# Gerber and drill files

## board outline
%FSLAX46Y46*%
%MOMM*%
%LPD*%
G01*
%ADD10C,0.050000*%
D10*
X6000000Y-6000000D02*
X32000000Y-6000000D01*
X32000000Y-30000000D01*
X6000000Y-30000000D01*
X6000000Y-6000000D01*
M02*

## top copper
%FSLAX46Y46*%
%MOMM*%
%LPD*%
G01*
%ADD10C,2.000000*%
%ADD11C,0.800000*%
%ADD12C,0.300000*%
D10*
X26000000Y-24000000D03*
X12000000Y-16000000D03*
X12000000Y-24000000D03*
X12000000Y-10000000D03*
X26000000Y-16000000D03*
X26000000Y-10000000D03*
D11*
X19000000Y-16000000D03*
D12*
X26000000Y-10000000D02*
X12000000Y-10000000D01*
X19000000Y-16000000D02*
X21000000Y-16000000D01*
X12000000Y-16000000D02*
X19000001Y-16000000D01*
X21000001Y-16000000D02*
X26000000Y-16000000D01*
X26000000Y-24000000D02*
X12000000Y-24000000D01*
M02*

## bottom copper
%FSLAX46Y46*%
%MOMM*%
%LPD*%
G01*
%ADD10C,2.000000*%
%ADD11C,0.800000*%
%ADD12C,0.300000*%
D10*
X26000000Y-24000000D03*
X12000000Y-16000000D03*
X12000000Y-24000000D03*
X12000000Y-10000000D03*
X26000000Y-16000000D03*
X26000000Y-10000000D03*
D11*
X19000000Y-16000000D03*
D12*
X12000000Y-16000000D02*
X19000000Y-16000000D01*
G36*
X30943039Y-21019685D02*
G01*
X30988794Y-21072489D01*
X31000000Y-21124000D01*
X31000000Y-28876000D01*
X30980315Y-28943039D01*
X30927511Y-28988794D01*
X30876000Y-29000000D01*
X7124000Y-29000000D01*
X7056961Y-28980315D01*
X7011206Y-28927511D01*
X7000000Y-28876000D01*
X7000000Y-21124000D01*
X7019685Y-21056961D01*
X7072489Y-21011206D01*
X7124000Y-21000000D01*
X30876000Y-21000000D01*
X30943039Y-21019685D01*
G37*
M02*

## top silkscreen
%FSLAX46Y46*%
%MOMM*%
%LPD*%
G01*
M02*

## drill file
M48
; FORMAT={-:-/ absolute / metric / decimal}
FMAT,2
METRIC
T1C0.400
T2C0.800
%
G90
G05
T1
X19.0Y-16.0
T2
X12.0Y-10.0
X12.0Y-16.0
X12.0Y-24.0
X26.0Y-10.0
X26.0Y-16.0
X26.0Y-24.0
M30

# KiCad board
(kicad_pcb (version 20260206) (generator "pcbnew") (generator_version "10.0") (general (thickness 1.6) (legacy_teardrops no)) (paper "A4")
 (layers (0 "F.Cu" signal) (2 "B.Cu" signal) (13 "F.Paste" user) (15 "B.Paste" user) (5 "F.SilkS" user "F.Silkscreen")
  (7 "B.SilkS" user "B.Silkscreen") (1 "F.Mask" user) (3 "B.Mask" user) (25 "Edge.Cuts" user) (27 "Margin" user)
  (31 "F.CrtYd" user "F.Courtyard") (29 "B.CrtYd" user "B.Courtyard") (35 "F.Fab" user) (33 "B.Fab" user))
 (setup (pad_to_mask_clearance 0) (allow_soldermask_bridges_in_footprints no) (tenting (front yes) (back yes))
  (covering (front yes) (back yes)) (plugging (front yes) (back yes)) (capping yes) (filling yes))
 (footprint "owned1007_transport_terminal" (layer "F.Cu") (at 26 24)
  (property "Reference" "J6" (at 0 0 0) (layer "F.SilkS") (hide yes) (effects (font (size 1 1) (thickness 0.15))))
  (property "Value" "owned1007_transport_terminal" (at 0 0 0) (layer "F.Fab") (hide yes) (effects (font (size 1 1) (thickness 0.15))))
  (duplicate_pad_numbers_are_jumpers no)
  (pad "1" thru_hole circle (at 0 0) (size 2 2) (drill 0.8) (layers "*.Cu" "*.Mask") (remove_unused_layers no) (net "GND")))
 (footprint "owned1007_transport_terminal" (layer "F.Cu") (at 12 16)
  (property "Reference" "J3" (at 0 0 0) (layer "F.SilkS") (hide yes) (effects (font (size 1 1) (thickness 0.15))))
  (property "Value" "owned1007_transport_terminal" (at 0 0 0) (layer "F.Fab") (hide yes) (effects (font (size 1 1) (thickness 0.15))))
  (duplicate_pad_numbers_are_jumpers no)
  (pad "1" thru_hole circle (at 0 0) (size 2 2) (drill 0.8) (layers "*.Cu" "*.Mask") (remove_unused_layers no) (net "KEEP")))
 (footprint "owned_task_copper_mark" (layer "F.Cu") (at 10 28)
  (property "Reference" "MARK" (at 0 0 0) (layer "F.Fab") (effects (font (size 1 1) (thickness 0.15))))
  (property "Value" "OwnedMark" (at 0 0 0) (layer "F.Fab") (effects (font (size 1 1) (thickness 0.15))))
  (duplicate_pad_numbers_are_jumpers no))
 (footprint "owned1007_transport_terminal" (layer "F.Cu") (at 12 24)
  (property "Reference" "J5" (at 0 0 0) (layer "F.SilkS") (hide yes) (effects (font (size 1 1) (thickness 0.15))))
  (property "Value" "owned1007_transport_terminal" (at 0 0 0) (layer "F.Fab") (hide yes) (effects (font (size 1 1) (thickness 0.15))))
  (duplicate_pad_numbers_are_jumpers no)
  (pad "1" thru_hole circle (at 0 0) (size 2 2) (drill 0.8) (layers "*.Cu" "*.Mask") (remove_unused_layers no) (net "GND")))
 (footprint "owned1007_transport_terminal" (layer "F.Cu") (at 12 10)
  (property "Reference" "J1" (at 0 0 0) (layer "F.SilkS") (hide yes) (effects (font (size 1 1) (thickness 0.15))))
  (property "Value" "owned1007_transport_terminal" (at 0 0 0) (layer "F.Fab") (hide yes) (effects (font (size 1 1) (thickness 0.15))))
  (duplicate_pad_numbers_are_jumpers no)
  (pad "1" thru_hole circle (at 0 0) (size 2 2) (drill 0.8) (layers "*.Cu" "*.Mask") (remove_unused_layers no) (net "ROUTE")))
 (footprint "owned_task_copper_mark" (layer "F.Cu") (at 13 28)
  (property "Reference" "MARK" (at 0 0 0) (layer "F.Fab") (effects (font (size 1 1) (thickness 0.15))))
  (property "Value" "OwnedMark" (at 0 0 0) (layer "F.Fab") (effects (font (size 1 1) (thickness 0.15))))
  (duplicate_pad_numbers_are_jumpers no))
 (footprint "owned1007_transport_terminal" (layer "F.Cu") (at 26 16)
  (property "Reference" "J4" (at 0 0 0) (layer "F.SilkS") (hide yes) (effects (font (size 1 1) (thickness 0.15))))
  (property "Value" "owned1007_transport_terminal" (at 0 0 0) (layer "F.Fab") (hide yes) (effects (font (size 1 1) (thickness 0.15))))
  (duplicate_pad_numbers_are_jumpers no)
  (pad "1" thru_hole circle (at 0 0) (size 2 2) (drill 0.8) (layers "*.Cu" "*.Mask") (remove_unused_layers no) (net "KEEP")))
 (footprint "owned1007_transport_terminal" (layer "F.Cu") (at 26 10)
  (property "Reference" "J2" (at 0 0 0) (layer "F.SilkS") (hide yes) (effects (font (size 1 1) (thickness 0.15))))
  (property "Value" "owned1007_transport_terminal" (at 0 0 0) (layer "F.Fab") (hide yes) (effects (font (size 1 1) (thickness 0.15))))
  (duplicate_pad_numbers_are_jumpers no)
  (pad "1" thru_hole circle (at 0 0) (size 2 2) (drill 0.8) (layers "*.Cu" "*.Mask") (remove_unused_layers no) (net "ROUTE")))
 (gr_rect (start 6 6) (end 32 30) (stroke (width 0.05) (type default)) (fill no) (layer "Edge.Cuts"))
 (segment (start 26 10) (end 12 10) (width 0.3) (layer "F.Cu") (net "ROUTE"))
 (segment (start 19 16) (end 21 16) (width 0.3) (layer "F.Cu") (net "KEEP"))
 (segment (start 12 16) (end 19.000001 16) (width 0.3) (layer "F.Cu") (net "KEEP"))
 (segment (start 21.000001 16) (end 26 16) (width 0.3) (layer "F.Cu") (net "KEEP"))
 (via (at 19 16) (size 0.8) (drill 0.4) (layers "F.Cu" "B.Cu") (free yes) (capping no) (covering (front no) (back no))
  (plugging (front no) (back no)) (filling no) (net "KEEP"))
 (segment (start 12 16) (end 19 16) (width 0.3) (locked yes) (layer "B.Cu") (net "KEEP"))
 (segment (start 26 24) (end 12 24) (width 0.3) (layer "F.Cu") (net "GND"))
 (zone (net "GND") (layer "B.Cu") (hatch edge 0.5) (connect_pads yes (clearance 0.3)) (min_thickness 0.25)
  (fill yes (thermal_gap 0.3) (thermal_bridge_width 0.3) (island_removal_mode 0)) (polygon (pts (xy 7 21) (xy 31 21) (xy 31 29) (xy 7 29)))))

